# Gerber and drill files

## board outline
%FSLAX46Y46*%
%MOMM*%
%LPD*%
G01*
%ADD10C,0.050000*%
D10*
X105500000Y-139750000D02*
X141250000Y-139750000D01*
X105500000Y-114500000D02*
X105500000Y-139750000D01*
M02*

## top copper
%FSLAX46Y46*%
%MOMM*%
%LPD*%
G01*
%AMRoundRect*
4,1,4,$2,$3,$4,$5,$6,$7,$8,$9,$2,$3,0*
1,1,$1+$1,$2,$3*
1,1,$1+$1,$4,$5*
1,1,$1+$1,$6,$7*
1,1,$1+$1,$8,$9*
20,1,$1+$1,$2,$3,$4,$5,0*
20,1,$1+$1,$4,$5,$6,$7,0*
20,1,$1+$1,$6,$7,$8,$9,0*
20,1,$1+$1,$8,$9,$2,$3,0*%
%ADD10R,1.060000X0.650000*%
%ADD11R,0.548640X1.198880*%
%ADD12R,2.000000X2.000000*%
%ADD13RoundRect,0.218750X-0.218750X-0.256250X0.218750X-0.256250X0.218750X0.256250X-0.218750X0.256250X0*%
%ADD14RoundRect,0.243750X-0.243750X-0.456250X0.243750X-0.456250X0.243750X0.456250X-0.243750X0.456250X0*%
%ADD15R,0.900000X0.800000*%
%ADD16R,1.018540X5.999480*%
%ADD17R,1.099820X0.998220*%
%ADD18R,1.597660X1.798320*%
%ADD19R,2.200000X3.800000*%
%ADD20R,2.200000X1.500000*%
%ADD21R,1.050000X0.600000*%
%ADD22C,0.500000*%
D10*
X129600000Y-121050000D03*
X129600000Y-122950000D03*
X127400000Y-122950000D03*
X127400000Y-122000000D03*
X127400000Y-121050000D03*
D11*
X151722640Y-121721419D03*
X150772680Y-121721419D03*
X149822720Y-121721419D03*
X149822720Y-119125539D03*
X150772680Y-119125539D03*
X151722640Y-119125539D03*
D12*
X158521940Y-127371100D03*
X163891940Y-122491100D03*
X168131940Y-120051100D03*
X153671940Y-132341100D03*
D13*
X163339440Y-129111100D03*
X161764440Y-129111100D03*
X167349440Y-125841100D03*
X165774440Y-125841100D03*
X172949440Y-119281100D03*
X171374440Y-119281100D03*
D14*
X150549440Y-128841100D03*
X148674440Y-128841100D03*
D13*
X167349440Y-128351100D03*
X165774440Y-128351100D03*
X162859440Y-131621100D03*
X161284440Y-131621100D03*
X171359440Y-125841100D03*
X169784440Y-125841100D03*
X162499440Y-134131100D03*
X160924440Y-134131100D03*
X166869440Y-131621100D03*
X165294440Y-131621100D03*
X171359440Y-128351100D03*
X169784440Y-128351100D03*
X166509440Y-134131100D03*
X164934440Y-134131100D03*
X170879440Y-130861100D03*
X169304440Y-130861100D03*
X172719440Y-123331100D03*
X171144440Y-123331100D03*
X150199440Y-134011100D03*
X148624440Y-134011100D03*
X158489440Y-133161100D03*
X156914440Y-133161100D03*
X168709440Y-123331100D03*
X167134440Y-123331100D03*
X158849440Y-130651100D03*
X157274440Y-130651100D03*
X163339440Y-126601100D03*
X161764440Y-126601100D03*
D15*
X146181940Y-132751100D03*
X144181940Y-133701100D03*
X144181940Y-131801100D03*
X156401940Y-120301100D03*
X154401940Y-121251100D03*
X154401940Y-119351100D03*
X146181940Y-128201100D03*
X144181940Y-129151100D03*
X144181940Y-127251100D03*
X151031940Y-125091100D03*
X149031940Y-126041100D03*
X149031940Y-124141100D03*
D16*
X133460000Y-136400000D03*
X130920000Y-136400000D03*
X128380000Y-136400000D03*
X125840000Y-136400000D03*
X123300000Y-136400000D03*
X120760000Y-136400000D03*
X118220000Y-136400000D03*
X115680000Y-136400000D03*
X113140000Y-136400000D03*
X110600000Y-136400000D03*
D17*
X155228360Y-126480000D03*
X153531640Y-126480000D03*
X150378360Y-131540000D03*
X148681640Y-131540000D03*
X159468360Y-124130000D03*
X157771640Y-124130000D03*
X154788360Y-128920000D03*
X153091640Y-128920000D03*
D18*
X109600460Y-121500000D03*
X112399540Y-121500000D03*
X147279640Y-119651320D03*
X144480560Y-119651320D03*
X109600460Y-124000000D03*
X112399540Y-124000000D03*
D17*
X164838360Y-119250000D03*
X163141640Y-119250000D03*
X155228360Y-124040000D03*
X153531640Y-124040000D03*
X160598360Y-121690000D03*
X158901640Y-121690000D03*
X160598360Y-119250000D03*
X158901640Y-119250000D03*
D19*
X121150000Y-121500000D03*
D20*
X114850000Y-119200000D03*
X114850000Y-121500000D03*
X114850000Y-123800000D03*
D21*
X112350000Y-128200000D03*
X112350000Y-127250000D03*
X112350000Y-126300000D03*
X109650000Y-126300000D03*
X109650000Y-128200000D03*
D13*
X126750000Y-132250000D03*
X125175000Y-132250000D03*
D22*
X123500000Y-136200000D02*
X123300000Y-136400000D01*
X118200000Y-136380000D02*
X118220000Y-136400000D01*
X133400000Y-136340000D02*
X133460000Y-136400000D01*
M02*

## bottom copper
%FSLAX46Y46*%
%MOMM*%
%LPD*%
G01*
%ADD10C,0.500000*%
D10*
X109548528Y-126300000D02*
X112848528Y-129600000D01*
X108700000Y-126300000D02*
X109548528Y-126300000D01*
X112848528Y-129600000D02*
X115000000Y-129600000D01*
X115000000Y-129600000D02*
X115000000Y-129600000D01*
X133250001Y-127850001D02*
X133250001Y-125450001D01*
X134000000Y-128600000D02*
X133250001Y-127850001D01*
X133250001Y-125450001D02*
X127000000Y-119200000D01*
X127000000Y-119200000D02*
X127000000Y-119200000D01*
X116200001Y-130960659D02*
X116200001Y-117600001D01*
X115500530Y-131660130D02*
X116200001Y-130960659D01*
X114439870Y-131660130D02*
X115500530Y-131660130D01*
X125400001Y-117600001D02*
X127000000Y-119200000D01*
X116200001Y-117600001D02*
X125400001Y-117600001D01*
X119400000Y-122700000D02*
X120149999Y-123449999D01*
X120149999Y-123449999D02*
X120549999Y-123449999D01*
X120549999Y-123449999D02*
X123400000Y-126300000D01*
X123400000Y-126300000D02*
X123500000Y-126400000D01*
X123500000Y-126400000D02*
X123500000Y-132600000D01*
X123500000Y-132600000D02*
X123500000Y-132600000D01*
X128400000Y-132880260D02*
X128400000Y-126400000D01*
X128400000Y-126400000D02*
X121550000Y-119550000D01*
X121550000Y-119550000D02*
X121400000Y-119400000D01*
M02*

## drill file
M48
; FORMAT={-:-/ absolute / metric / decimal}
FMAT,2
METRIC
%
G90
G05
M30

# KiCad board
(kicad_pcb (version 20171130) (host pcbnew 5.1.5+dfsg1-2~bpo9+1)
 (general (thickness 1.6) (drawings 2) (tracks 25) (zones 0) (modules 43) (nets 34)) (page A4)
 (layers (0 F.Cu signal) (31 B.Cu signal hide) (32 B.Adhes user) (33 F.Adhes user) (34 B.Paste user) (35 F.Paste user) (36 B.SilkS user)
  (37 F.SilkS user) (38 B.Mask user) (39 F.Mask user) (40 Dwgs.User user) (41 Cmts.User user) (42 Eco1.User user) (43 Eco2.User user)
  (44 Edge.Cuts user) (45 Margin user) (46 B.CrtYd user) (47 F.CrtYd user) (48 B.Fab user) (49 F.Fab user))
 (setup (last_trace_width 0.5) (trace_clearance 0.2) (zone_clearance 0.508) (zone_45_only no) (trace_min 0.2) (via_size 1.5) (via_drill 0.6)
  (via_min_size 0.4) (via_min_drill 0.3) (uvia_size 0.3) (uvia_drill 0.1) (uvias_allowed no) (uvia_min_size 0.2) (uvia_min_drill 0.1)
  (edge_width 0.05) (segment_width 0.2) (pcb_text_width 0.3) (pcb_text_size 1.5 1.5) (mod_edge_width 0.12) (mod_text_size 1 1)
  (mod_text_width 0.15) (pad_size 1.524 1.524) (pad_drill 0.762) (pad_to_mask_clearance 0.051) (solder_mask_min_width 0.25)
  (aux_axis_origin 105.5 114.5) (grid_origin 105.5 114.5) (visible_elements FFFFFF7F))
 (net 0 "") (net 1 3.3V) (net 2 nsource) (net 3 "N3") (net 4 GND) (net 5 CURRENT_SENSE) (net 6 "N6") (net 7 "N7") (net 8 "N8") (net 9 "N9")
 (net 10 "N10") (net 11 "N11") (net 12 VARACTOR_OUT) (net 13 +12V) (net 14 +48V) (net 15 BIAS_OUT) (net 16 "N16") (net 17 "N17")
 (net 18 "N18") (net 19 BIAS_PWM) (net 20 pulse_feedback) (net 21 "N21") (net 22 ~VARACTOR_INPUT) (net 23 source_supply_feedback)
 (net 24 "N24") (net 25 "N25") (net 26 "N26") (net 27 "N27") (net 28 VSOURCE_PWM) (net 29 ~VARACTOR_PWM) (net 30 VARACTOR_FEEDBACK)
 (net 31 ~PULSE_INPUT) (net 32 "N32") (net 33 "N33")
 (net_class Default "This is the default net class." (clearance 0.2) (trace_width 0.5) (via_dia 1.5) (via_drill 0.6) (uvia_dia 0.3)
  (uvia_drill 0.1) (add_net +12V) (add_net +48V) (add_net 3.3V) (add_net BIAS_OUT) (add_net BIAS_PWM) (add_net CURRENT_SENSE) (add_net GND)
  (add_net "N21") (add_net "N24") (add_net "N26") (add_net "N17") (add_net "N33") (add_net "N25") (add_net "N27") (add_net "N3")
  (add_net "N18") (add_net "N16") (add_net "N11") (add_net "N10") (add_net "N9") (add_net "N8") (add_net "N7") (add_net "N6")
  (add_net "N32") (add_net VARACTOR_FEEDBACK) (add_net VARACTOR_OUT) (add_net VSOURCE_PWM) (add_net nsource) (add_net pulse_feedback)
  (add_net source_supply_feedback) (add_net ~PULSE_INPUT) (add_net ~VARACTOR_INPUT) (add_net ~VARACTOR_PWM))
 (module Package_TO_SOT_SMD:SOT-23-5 (layer F.Cu) (at 128.5 122)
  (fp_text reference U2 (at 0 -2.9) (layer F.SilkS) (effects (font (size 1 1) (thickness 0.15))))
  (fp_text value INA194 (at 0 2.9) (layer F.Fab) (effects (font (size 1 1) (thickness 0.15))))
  (pad 5 smd rect (at 1.1 -0.95) (size 1.06 0.65) (layers F.Cu F.Paste F.Mask) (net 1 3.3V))
  (pad 4 smd rect (at 1.1 0.95) (size 1.06 0.65) (layers F.Cu F.Paste F.Mask) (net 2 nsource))
  (pad 3 smd rect (at -1.1 0.95) (size 1.06 0.65) (layers F.Cu F.Paste F.Mask) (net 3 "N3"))
  (pad 2 smd rect (at -1.1 0) (size 1.06 0.65) (layers F.Cu F.Paste F.Mask) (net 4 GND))
  (pad 1 smd rect (at -1.1 -0.95) (size 1.06 0.65) (layers F.Cu F.Paste F.Mask) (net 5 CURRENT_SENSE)))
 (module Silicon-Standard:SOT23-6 (layer F.Cu) (at 150.77268 120.423479)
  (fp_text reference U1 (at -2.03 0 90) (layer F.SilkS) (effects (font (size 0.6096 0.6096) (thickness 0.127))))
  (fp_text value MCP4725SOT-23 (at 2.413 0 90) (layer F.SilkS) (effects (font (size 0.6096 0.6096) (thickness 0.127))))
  (pad 6 smd rect (at 0.94996 1.29794) (size 0.54864 1.19888) (layers F.Cu F.Paste F.Mask) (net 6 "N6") (solder_mask_margin 0.1016))
  (pad 5 smd rect (at 0 1.29794) (size 0.54864 1.19888) (layers F.Cu F.Paste F.Mask) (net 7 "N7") (solder_mask_margin 0.1016))
  (pad 4 smd rect (at -0.94996 1.29794) (size 0.54864 1.19888) (layers F.Cu F.Paste F.Mask) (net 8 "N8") (solder_mask_margin 0.1016))
  (pad 3 smd rect (at -0.94996 -1.29794) (size 0.54864 1.19888) (layers F.Cu F.Paste F.Mask) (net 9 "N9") (solder_mask_margin 0.1016))
  (pad 2 smd rect (at 0 -1.29794 180) (size 0.54864 1.19888) (layers F.Cu F.Paste F.Mask) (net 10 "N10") (solder_mask_margin 0.1016))
  (pad 1 smd rect (at 0.94996 -1.29794) (size 0.54864 1.19888) (layers F.Cu F.Paste F.Mask) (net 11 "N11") (solder_mask_margin 0.1016)))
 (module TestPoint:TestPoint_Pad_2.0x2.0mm (layer F.Cu) (at 158.52194 127.3711)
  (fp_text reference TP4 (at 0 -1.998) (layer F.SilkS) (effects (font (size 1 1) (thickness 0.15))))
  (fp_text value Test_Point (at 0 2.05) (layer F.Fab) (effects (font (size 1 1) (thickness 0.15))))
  (pad 1 smd rect (at 0 0) (size 2 2) (layers F.Cu F.Mask) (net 2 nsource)))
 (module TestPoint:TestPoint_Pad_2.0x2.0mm (layer F.Cu) (at 163.89194 122.4911)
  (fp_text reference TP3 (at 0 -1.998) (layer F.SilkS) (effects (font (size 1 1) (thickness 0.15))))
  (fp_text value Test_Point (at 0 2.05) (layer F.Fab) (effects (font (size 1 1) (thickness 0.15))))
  (pad 1 smd rect (at 0 0) (size 2 2) (layers F.Cu F.Mask) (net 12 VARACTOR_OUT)))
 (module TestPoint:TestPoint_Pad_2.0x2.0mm (layer F.Cu) (at 168.13194 120.0511)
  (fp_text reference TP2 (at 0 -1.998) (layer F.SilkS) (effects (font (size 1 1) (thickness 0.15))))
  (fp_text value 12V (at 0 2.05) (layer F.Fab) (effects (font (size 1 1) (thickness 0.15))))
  (pad 1 smd rect (at 0 0) (size 2 2) (layers F.Cu F.Mask) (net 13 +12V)))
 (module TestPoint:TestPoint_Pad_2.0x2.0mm (layer F.Cu) (at 153.67194 132.3411)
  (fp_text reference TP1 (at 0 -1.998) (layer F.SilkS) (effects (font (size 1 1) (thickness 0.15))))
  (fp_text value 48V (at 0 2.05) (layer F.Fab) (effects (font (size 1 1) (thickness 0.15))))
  (pad 1 smd rect (at 0 0) (size 2 2) (layers F.Cu F.Mask) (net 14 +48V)))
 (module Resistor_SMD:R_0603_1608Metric (layer F.Cu) (at 162.55194 129.1111)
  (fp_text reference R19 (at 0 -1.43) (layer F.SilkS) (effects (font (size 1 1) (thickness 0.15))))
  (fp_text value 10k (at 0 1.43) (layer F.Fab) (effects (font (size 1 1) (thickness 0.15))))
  (pad 2 smd roundrect (at 0.7875 0) (size 0.875 0.95) (layers F.Cu F.Paste F.Mask) (roundrect_rratio 0.25) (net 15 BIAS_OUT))
  (pad 1 smd roundrect (at -0.7875 0) (size 0.875 0.95) (layers F.Cu F.Paste F.Mask) (roundrect_rratio 0.25) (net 4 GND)))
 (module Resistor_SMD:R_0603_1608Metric (layer F.Cu) (at 166.56194 125.8411)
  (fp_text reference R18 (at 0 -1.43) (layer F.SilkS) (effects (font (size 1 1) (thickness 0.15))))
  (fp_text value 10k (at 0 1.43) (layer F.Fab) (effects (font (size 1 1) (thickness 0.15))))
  (pad 2 smd roundrect (at 0.7875 0) (size 0.875 0.95) (layers F.Cu F.Paste F.Mask) (roundrect_rratio 0.25) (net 2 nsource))
  (pad 1 smd roundrect (at -0.7875 0) (size 0.875 0.95) (layers F.Cu F.Paste F.Mask) (roundrect_rratio 0.25) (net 15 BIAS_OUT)))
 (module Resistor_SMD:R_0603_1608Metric (layer F.Cu) (at 172.16194 119.2811)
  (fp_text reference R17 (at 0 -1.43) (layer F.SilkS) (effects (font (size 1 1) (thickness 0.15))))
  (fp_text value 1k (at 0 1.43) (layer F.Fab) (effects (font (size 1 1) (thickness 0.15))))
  (pad 2 smd roundrect (at 0.7875 0) (size 0.875 0.95) (layers F.Cu F.Paste F.Mask) (roundrect_rratio 0.25) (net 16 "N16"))
  (pad 1 smd roundrect (at -0.7875 0) (size 0.875 0.95) (layers F.Cu F.Paste F.Mask) (roundrect_rratio 0.25) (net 4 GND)))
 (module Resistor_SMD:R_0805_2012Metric (layer F.Cu) (at 149.61194 128.8411)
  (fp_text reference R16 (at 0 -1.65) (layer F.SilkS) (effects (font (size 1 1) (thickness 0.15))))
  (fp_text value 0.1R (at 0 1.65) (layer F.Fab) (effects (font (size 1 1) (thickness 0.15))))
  (pad 2 smd roundrect (at 0.9375 0) (size 0.975 1.4) (layers F.Cu F.Paste F.Mask) (roundrect_rratio 0.25) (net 3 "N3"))
  (pad 1 smd roundrect (at -0.9375 0) (size 0.975 1.4) (layers F.Cu F.Paste F.Mask) (roundrect_rratio 0.25) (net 2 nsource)))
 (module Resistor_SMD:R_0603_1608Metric (layer F.Cu) (at 166.56194 128.3511)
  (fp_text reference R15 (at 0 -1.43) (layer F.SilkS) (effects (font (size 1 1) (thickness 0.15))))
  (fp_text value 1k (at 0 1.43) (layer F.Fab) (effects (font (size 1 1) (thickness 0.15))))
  (pad 2 smd roundrect (at 0.7875 0) (size 0.875 0.95) (layers F.Cu F.Paste F.Mask) (roundrect_rratio 0.25) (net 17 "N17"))
  (pad 1 smd roundrect (at -0.7875 0) (size 0.875 0.95) (layers F.Cu F.Paste F.Mask) (roundrect_rratio 0.25) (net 16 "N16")))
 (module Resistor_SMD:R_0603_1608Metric (layer F.Cu) (at 162.07194 131.6211)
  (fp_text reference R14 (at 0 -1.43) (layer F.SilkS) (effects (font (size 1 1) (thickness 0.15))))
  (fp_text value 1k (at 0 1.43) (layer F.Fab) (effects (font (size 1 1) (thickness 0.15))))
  (pad 2 smd roundrect (at 0.7875 0) (size 0.875 0.95) (layers F.Cu F.Paste F.Mask) (roundrect_rratio 0.25) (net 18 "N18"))
  (pad 1 smd roundrect (at -0.7875 0) (size 0.875 0.95) (layers F.Cu F.Paste F.Mask) (roundrect_rratio 0.25) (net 17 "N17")))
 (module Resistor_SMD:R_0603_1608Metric (layer F.Cu) (at 170.57194 125.8411)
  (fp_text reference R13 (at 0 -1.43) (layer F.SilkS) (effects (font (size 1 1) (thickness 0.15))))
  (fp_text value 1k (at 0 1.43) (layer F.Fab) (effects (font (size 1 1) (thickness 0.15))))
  (pad 2 smd roundrect (at 0.7875 0) (size 0.875 0.95) (layers F.Cu F.Paste F.Mask) (roundrect_rratio 0.25) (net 1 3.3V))
  (pad 1 smd roundrect (at -0.7875 0) (size 0.875 0.95) (layers F.Cu F.Paste F.Mask) (roundrect_rratio 0.25) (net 18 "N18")))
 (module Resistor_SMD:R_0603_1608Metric (layer F.Cu) (at 161.71194 134.1311)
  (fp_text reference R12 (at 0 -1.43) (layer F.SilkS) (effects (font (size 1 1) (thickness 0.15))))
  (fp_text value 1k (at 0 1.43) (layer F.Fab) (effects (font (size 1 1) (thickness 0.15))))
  (pad 2 smd roundrect (at 0.7875 0) (size 0.875 0.95) (layers F.Cu F.Paste F.Mask) (roundrect_rratio 0.25) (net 17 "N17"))
  (pad 1 smd roundrect (at -0.7875 0) (size 0.875 0.95) (layers F.Cu F.Paste F.Mask) (roundrect_rratio 0.25) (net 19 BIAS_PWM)))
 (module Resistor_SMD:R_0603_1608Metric (layer F.Cu) (at 166.08194 131.6211)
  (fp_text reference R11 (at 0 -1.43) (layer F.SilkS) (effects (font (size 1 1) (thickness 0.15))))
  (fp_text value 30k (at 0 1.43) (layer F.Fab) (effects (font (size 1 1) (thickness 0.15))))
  (pad 2 smd roundrect (at 0.7875 0) (size 0.875 0.95) (layers F.Cu F.Paste F.Mask) (roundrect_rratio 0.25) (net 12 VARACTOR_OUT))
  (pad 1 smd roundrect (at -0.7875 0) (size 0.875 0.95) (layers F.Cu F.Paste F.Mask) (roundrect_rratio 0.25) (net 4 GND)))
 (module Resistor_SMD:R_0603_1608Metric (layer F.Cu) (at 170.57194 128.3511)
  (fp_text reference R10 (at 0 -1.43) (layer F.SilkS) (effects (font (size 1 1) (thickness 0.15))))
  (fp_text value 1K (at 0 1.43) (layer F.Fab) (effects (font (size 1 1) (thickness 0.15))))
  (pad 2 smd roundrect (at 0.7875 0) (size 0.875 0.95) (layers F.Cu F.Paste F.Mask) (roundrect_rratio 0.25) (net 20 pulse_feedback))
  (pad 1 smd roundrect (at -0.7875 0) (size 0.875 0.95) (layers F.Cu F.Paste F.Mask) (roundrect_rratio 0.25) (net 4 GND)))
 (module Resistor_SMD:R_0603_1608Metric (layer F.Cu) (at 165.72194 134.1311)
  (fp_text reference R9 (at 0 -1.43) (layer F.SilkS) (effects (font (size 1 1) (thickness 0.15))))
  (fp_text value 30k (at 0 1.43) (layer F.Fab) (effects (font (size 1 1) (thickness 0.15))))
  (pad 2 smd roundrect (at 0.7875 0) (size 0.875 0.95) (layers F.Cu F.Paste F.Mask) (roundrect_rratio 0.25) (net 14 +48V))
  (pad 1 smd roundrect (at -0.7875 0) (size 0.875 0.95) (layers F.Cu F.Paste F.Mask) (roundrect_rratio 0.25) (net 12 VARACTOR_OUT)))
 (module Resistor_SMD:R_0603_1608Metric (layer F.Cu) (at 170.09194 130.8611)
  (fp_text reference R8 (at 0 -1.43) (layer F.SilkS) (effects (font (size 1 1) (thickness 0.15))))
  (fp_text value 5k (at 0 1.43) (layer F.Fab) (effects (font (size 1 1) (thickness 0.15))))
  (pad 2 smd roundrect (at 0.7875 0) (size 0.875 0.95) (layers F.Cu F.Paste F.Mask) (roundrect_rratio 0.25) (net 2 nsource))
  (pad 1 smd roundrect (at -0.7875 0) (size 0.875 0.95) (layers F.Cu F.Paste F.Mask) (roundrect_rratio 0.25) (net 20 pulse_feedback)))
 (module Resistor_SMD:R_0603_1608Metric (layer F.Cu) (at 171.93194 123.3311)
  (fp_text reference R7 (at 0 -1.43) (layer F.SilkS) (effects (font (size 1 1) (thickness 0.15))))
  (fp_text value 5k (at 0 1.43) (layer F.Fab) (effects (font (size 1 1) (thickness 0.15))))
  (pad 2 smd roundrect (at 0.7875 0) (size 0.875 0.95) (layers F.Cu F.Paste F.Mask) (roundrect_rratio 0.25) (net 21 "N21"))
  (pad 1 smd roundrect (at -0.7875 0) (size 0.875 0.95) (layers F.Cu F.Paste F.Mask) (roundrect_rratio 0.25) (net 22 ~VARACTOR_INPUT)))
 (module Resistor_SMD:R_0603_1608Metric (layer F.Cu) (at 149.41194 134.0111)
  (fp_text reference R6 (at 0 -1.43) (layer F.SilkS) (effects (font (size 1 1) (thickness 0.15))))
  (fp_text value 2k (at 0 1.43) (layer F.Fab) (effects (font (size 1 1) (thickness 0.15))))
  (pad 2 smd roundrect (at 0.7875 0) (size 0.875 0.95) (layers F.Cu F.Paste F.Mask) (roundrect_rratio 0.25) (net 21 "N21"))
  (pad 1 smd roundrect (at -0.7875 0) (size 0.875 0.95) (layers F.Cu F.Paste F.Mask) (roundrect_rratio 0.25) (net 4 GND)))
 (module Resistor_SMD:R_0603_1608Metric (layer F.Cu) (at 157.70194 133.1611)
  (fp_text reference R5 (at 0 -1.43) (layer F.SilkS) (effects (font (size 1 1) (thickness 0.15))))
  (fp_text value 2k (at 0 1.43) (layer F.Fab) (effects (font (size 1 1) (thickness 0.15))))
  (pad 2 smd roundrect (at 0.7875 0) (size 0.875 0.95) (layers F.Cu F.Paste F.Mask) (roundrect_rratio 0.25) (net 1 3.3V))
  (pad 1 smd roundrect (at -0.7875 0) (size 0.875 0.95) (layers F.Cu F.Paste F.Mask) (roundrect_rratio 0.25) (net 21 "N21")))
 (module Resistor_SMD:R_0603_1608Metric (layer F.Cu) (at 167.92194 123.3311)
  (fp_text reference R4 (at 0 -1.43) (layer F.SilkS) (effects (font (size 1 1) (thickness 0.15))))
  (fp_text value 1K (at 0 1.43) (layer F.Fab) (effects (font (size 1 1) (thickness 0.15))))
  (pad 2 smd roundrect (at 0.7875 0) (size 0.875 0.95) (layers F.Cu F.Paste F.Mask) (roundrect_rratio 0.25) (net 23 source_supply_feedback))
  (pad 1 smd roundrect (at -0.7875 0) (size 0.875 0.95) (layers F.Cu F.Paste F.Mask) (roundrect_rratio 0.25) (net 4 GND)))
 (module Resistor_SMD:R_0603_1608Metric (layer F.Cu) (at 158.06194 130.6511)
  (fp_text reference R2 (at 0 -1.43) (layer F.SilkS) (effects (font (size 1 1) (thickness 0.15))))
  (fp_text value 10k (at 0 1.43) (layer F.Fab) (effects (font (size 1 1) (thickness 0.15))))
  (pad 2 smd roundrect (at 0.7875 0) (size 0.875 0.95) (layers F.Cu F.Paste F.Mask) (roundrect_rratio 0.25) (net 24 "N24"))
  (pad 1 smd roundrect (at -0.7875 0) (size 0.875 0.95) (layers F.Cu F.Paste F.Mask) (roundrect_rratio 0.25) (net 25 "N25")))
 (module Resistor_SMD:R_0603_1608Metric (layer F.Cu) (at 162.55194 126.6011)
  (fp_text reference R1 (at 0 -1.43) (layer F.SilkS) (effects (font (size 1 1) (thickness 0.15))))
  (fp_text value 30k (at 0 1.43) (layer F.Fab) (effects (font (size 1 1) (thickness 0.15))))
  (pad 2 smd roundrect (at 0.7875 0) (size 0.875 0.95) (layers F.Cu F.Paste F.Mask) (roundrect_rratio 0.25) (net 13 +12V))
  (pad 1 smd roundrect (at -0.7875 0) (size 0.875 0.95) (layers F.Cu F.Paste F.Mask) (roundrect_rratio 0.25) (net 24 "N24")))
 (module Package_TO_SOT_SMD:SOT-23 (layer F.Cu) (at 145.18194 132.7511)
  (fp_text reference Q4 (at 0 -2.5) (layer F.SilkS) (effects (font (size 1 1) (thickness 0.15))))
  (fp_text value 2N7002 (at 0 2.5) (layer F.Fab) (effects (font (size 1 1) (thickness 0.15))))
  (pad 3 smd rect (at 1 0) (size 0.9 0.8) (layers F.Cu F.Paste F.Mask) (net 15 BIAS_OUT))
  (pad 2 smd rect (at -1 0.95) (size 0.9 0.8) (layers F.Cu F.Paste F.Mask) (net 4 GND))
  (pad 1 smd rect (at -1 -0.95) (size 0.9 0.8) (layers F.Cu F.Paste F.Mask) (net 17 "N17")))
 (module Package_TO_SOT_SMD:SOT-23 (layer F.Cu) (at 155.40194 120.3011)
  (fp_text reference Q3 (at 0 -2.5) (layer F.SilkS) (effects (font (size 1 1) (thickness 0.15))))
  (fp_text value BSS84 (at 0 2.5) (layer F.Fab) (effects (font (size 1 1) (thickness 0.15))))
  (pad 3 smd rect (at 1 0) (size 0.9 0.8) (layers F.Cu F.Paste F.Mask) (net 3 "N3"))
  (pad 2 smd rect (at -1 0.95) (size 0.9 0.8) (layers F.Cu F.Paste F.Mask) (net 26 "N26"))
  (pad 1 smd rect (at -1 -0.95) (size 0.9 0.8) (layers F.Cu F.Paste F.Mask) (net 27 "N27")))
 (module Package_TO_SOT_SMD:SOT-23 (layer F.Cu) (at 145.18194 128.2011)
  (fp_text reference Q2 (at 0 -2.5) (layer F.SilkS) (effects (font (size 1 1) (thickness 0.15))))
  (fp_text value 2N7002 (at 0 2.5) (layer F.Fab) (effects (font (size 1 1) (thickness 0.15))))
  (pad 3 smd rect (at 1 0) (size 0.9 0.8) (layers F.Cu F.Paste F.Mask) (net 25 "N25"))
  (pad 2 smd rect (at -1 0.95) (size 0.9 0.8) (layers F.Cu F.Paste F.Mask) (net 4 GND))
  (pad 1 smd rect (at -1 -0.95) (size 0.9 0.8) (layers F.Cu F.Paste F.Mask) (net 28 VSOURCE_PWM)))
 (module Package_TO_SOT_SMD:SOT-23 (layer F.Cu) (at 150.03194 125.0911)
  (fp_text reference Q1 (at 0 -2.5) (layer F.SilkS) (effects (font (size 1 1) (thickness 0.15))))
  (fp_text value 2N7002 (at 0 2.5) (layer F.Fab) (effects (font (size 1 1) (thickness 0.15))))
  (pad 3 smd rect (at 1 0) (size 0.9 0.8) (layers F.Cu F.Paste F.Mask) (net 12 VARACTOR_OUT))
  (pad 2 smd rect (at -1 0.95) (size 0.9 0.8) (layers F.Cu F.Paste F.Mask) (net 4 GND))
  (pad 1 smd rect (at -1 -0.95) (size 0.9 0.8) (layers F.Cu F.Paste F.Mask) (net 21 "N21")))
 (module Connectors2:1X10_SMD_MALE (layer F.Cu) (at 110.6 136.4)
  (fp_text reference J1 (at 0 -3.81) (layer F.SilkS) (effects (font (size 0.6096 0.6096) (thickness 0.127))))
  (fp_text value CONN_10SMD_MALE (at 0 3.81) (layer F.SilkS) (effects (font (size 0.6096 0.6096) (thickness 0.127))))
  (pad 10 smd rect (at 22.86 0) (size 1.01854 5.99948) (layers F.Cu F.Paste F.Mask) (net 19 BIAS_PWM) (solder_mask_margin 0.1016))
  (pad 9 smd rect (at 20.32 0) (size 1.01854 5.99948) (layers F.Cu F.Paste F.Mask) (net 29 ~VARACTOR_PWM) (solder_mask_margin 0.1016))
  (pad 8 smd rect (at 17.78 0) (size 1.01854 5.99948) (layers F.Cu F.Paste F.Mask) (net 5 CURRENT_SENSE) (solder_mask_margin 0.1016))
  (pad 7 smd rect (at 15.24 0) (size 1.01854 5.99948) (layers F.Cu F.Paste F.Mask) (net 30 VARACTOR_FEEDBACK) (solder_mask_margin 0.1016))
  (pad 6 smd rect (at 12.7 0) (size 1.01854 5.99948) (layers F.Cu F.Paste F.Mask) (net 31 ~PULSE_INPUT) (solder_mask_margin 0.1016))
  (pad 5 smd rect (at 10.16 0) (size 1.01854 5.99948) (layers F.Cu F.Paste F.Mask) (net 20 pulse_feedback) (solder_mask_margin 0.1016))
  (pad 4 smd rect (at 7.62 0) (size 1.01854 5.99948) (layers F.Cu F.Paste F.Mask) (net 23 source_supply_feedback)
   (solder_mask_margin 0.1016))
  (pad 3 smd rect (at 5.08 0) (size 1.01854 5.99948) (layers F.Cu F.Paste F.Mask) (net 1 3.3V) (solder_mask_margin 0.1016))
  (pad 2 smd rect (at 2.54 0) (size 1.01854 5.99948) (layers F.Cu F.Paste F.Mask) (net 28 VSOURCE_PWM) (solder_mask_margin 0.1016))
  (pad 1 smd rect (at 0 0) (size 1.01854 5.99948) (layers F.Cu F.Paste F.Mask) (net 4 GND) (solder_mask_margin 0.1016)))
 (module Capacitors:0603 (layer F.Cu) (at 154.38 126.48)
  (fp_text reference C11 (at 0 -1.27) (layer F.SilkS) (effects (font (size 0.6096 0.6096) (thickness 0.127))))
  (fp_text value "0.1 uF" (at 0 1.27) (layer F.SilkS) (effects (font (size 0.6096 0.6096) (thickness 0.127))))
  (pad 2 smd rect (at 0.84836 0) (size 1.09982 0.99822) (layers F.Cu F.Paste F.Mask) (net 15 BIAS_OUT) (solder_mask_margin 0.1016))
  (pad 1 smd rect (at -0.84836 0) (size 1.09982 0.99822) (layers F.Cu F.Paste F.Mask) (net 4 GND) (solder_mask_margin 0.1016)))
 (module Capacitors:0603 (layer F.Cu) (at 149.53 131.54)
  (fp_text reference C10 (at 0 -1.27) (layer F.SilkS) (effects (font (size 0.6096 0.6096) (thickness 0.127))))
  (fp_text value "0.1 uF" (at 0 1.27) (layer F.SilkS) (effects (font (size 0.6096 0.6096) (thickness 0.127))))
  (pad 2 smd rect (at 0.84836 0) (size 1.09982 0.99822) (layers F.Cu F.Paste F.Mask) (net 1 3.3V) (solder_mask_margin 0.1016))
  (pad 1 smd rect (at -0.84836 0) (size 1.09982 0.99822) (layers F.Cu F.Paste F.Mask) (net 4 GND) (solder_mask_margin 0.1016)))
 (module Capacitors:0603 (layer F.Cu) (at 158.62 124.13)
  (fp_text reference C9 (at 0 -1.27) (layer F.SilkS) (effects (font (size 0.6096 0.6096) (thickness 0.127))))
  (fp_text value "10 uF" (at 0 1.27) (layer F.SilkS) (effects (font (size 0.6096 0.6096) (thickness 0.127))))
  (pad 2 smd rect (at 0.84836 0) (size 1.09982 0.99822) (layers F.Cu F.Paste F.Mask) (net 17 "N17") (solder_mask_margin 0.1016))
  (pad 1 smd rect (at -0.84836 0) (size 1.09982 0.99822) (layers F.Cu F.Paste F.Mask) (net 4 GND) (solder_mask_margin 0.1016)))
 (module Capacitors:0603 (layer F.Cu) (at 153.94 128.92)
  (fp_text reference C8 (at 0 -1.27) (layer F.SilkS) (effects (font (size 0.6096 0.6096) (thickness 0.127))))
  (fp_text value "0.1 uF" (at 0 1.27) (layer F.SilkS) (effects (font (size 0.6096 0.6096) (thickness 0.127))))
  (pad 2 smd rect (at 0.84836 0) (size 1.09982 0.99822) (layers F.Cu F.Paste F.Mask) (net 26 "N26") (solder_mask_margin 0.1016))
  (pad 1 smd rect (at -0.84836 0) (size 1.09982 0.99822) (layers F.Cu F.Paste F.Mask) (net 4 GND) (solder_mask_margin 0.1016)))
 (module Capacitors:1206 (layer F.Cu) (at 111 121.5 180)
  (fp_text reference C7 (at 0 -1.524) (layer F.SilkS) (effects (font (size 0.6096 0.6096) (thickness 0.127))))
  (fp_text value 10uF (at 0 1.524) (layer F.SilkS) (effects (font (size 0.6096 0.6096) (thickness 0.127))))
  (pad 2 smd rect (at 1.39954 0 180) (size 1.59766 1.79832) (layers F.Cu F.Paste F.Mask) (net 4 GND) (solder_mask_margin 0.1016))
  (pad 1 smd rect (at -1.39954 0 180) (size 1.59766 1.79832) (layers F.Cu F.Paste F.Mask) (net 26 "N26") (solder_mask_margin 0.1016)))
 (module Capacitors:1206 (layer F.Cu) (at 145.8801 119.65132)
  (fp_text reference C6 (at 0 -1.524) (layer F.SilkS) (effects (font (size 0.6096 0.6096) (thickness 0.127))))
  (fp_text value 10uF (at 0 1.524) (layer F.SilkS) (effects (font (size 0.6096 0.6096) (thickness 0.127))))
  (pad 2 smd rect (at 1.39954 0) (size 1.59766 1.79832) (layers F.Cu F.Paste F.Mask) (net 4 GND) (solder_mask_margin 0.1016))
  (pad 1 smd rect (at -1.39954 0) (size 1.59766 1.79832) (layers F.Cu F.Paste F.Mask) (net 24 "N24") (solder_mask_margin 0.1016)))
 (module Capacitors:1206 (layer F.Cu) (at 111 124 180)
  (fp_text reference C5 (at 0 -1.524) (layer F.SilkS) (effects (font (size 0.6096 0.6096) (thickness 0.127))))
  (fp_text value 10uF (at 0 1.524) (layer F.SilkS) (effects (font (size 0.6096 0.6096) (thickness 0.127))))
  (pad 2 smd rect (at 1.39954 0 180) (size 1.59766 1.79832) (layers F.Cu F.Paste F.Mask) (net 4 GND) (solder_mask_margin 0.1016))
  (pad 1 smd rect (at -1.39954 0 180) (size 1.59766 1.79832) (layers F.Cu F.Paste F.Mask) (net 13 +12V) (solder_mask_margin 0.1016)))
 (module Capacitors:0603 (layer F.Cu) (at 163.99 119.25)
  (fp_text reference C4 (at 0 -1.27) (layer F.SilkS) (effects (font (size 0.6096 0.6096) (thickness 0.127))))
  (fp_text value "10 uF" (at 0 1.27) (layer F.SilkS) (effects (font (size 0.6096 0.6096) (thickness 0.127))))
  (pad 2 smd rect (at 0.84836 0) (size 1.09982 0.99822) (layers F.Cu F.Paste F.Mask) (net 21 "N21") (solder_mask_margin 0.1016))
  (pad 1 smd rect (at -0.84836 0) (size 1.09982 0.99822) (layers F.Cu F.Paste F.Mask) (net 4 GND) (solder_mask_margin 0.1016)))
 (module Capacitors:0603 (layer F.Cu) (at 154.38 124.04)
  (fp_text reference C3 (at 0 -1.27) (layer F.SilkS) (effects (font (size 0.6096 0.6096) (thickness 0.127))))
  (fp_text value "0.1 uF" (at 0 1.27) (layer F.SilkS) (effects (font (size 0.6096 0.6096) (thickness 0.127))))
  (pad 2 smd rect (at 0.84836 0) (size 1.09982 0.99822) (layers F.Cu F.Paste F.Mask) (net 14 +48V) (solder_mask_margin 0.1016))
  (pad 1 smd rect (at -0.84836 0) (size 1.09982 0.99822) (layers F.Cu F.Paste F.Mask) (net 4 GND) (solder_mask_margin 0.1016)))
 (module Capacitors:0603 (layer F.Cu) (at 159.75 121.69)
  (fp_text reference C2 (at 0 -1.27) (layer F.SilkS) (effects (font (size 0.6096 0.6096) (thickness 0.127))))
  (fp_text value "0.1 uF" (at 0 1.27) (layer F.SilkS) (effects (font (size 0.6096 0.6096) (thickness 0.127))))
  (pad 2 smd rect (at 0.84836 0) (size 1.09982 0.99822) (layers F.Cu F.Paste F.Mask) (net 13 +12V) (solder_mask_margin 0.1016))
  (pad 1 smd rect (at -0.84836 0) (size 1.09982 0.99822) (layers F.Cu F.Paste F.Mask) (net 4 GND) (solder_mask_margin 0.1016)))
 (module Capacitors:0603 (layer F.Cu) (at 159.75 119.25)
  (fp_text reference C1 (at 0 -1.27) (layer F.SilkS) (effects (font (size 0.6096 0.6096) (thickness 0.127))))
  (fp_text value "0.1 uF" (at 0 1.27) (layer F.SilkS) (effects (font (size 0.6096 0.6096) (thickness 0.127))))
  (pad 2 smd rect (at 0.84836 0) (size 1.09982 0.99822) (layers F.Cu F.Paste F.Mask) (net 12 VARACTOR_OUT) (solder_mask_margin 0.1016))
  (pad 1 smd rect (at -0.84836 0) (size 1.09982 0.99822) (layers F.Cu F.Paste F.Mask) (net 4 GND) (solder_mask_margin 0.1016)))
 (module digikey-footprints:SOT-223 (layer F.Cu) (at 118 121.5 270)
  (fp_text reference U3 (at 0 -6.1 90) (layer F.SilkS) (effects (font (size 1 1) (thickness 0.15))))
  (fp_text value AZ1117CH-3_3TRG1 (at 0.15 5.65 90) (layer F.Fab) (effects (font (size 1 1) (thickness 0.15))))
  (pad 4 smd rect (at 0 -3.15 270) (size 3.8 2.2) (layers F.Cu F.Paste F.Mask) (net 26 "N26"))
  (pad 1 smd rect (at -2.3 3.15 270) (size 1.5 2.2) (layers F.Cu F.Paste F.Mask) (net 24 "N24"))
  (pad 2 smd rect (at 0 3.15 270) (size 1.5 2.2) (layers F.Cu F.Paste F.Mask) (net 26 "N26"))
  (pad 3 smd rect (at 2.3 3.15 270) (size 1.5 2.2) (layers F.Cu F.Paste F.Mask) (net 13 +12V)))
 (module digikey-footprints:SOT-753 (layer F.Cu) (at 111 127.25 90)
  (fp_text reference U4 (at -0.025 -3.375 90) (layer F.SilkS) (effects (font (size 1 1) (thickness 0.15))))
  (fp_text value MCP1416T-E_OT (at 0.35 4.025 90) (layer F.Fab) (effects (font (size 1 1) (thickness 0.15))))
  (pad 1 smd rect (at -0.95 1.35 90) (size 0.6 1.05) (layers F.Cu F.Paste F.Mask) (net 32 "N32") (solder_mask_margin 0.07))
  (pad 2 smd rect (at 0 1.35 90) (size 0.6 1.05) (layers F.Cu F.Paste F.Mask) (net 13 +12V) (solder_mask_margin 0.07))
  (pad 3 smd rect (at 0.95 1.35 90) (size 0.6 1.05) (layers F.Cu F.Paste F.Mask) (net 31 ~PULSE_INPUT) (solder_mask_margin 0.07))
  (pad 4 smd rect (at 0.95 -1.35 90) (size 0.6 1.05) (layers F.Cu F.Paste F.Mask) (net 4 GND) (solder_mask_margin 0.07))
  (pad 5 smd rect (at -0.95 -1.35 90) (size 0.6 1.05) (layers F.Cu F.Paste F.Mask) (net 27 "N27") (solder_mask_margin 0.07)))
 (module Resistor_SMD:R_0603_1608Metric (layer F.Cu) (at 125.9625 132.25)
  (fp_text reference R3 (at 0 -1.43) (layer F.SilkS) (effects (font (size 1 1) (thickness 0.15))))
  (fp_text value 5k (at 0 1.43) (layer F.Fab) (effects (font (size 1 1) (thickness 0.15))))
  (pad 2 smd roundrect (at 0.7875 0) (size 0.875 0.95) (layers F.Cu F.Paste F.Mask) (roundrect_rratio 0.25) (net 26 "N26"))
  (pad 1 smd roundrect (at -0.7875 0) (size 0.875 0.95) (layers F.Cu F.Paste F.Mask) (roundrect_rratio 0.25) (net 23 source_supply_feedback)))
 (gr_line (start 105.5 139.75) (end 141.25 139.75) (layer Edge.Cuts) (width 0.05))
 (gr_line (start 105.5 114.5) (end 105.5 139.75) (layer Edge.Cuts) (width 0.05))
 (segment (start 109.548528 126.3) (end 112.848528 129.6) (width 0.5) (layer B.Cu) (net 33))
 (segment (start 108.7 126.3) (end 109.548528 126.3) (width 0.5) (layer B.Cu) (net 33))
 (segment (start 112.848528 129.6) (end 115 129.6) (width 0.5) (layer B.Cu) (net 33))
 (segment (start 115 129.6) (end 115 129.6) (width 0.5) (layer B.Cu) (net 33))
 (segment (start 133.250001 127.850001) (end 133.250001 125.450001) (width 0.5) (layer B.Cu) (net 1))
 (segment (start 134 128.6) (end 133.250001 127.850001) (width 0.5) (layer B.Cu) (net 1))
 (segment (start 133.250001 125.450001) (end 127 119.2) (width 0.5) (layer B.Cu) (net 1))
 (segment (start 127 119.2) (end 127 119.2) (width 0.5) (layer B.Cu) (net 1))
 (segment (start 116.200001 130.960659) (end 116.200001 117.600001) (width 0.5) (layer B.Cu) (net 1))
 (segment (start 115.50053 131.66013) (end 116.200001 130.960659) (width 0.5) (layer B.Cu) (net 1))
 (segment (start 114.43987 131.66013) (end 115.50053 131.66013) (width 0.5) (layer B.Cu) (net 1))
 (segment (start 125.400001 117.600001) (end 127 119.2) (width 0.5) (layer B.Cu) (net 1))
 (segment (start 116.200001 117.600001) (end 125.400001 117.600001) (width 0.5) (layer B.Cu) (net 1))
 (segment (start 119.4 122.7) (end 120.149999 123.449999) (width 0.5) (layer B.Cu) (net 31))
 (segment (start 120.149999 123.449999) (end 120.549999 123.449999) (width 0.5) (layer B.Cu) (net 31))
 (segment (start 120.549999 123.449999) (end 123.4 126.3) (width 0.5) (layer B.Cu) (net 31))
 (segment (start 123.4 126.3) (end 123.5 126.4) (width 0.5) (layer B.Cu) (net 31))
 (segment (start 123.5 126.4) (end 123.5 132.6) (width 0.5) (layer B.Cu) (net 31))
 (segment (start 123.5 132.6) (end 123.5 132.6) (width 0.5) (layer B.Cu) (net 31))
 (segment (start 123.5 136.2) (end 123.3 136.4) (width 0.5) (layer F.Cu) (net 31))
 (segment (start 118.2 136.38) (end 118.22 136.4) (width 0.5) (layer F.Cu) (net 23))
 (segment (start 133.4 136.34) (end 133.46 136.4) (width 0.5) (layer F.Cu) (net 19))
 (segment (start 128.4 132.88026) (end 128.4 126.4) (width 0.5) (layer B.Cu) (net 5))
 (segment (start 128.4 126.4) (end 121.55 119.55) (width 0.5) (layer B.Cu) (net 5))
 (segment (start 121.55 119.55) (end 121.4 119.4) (width 0.5) (layer B.Cu) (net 5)))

